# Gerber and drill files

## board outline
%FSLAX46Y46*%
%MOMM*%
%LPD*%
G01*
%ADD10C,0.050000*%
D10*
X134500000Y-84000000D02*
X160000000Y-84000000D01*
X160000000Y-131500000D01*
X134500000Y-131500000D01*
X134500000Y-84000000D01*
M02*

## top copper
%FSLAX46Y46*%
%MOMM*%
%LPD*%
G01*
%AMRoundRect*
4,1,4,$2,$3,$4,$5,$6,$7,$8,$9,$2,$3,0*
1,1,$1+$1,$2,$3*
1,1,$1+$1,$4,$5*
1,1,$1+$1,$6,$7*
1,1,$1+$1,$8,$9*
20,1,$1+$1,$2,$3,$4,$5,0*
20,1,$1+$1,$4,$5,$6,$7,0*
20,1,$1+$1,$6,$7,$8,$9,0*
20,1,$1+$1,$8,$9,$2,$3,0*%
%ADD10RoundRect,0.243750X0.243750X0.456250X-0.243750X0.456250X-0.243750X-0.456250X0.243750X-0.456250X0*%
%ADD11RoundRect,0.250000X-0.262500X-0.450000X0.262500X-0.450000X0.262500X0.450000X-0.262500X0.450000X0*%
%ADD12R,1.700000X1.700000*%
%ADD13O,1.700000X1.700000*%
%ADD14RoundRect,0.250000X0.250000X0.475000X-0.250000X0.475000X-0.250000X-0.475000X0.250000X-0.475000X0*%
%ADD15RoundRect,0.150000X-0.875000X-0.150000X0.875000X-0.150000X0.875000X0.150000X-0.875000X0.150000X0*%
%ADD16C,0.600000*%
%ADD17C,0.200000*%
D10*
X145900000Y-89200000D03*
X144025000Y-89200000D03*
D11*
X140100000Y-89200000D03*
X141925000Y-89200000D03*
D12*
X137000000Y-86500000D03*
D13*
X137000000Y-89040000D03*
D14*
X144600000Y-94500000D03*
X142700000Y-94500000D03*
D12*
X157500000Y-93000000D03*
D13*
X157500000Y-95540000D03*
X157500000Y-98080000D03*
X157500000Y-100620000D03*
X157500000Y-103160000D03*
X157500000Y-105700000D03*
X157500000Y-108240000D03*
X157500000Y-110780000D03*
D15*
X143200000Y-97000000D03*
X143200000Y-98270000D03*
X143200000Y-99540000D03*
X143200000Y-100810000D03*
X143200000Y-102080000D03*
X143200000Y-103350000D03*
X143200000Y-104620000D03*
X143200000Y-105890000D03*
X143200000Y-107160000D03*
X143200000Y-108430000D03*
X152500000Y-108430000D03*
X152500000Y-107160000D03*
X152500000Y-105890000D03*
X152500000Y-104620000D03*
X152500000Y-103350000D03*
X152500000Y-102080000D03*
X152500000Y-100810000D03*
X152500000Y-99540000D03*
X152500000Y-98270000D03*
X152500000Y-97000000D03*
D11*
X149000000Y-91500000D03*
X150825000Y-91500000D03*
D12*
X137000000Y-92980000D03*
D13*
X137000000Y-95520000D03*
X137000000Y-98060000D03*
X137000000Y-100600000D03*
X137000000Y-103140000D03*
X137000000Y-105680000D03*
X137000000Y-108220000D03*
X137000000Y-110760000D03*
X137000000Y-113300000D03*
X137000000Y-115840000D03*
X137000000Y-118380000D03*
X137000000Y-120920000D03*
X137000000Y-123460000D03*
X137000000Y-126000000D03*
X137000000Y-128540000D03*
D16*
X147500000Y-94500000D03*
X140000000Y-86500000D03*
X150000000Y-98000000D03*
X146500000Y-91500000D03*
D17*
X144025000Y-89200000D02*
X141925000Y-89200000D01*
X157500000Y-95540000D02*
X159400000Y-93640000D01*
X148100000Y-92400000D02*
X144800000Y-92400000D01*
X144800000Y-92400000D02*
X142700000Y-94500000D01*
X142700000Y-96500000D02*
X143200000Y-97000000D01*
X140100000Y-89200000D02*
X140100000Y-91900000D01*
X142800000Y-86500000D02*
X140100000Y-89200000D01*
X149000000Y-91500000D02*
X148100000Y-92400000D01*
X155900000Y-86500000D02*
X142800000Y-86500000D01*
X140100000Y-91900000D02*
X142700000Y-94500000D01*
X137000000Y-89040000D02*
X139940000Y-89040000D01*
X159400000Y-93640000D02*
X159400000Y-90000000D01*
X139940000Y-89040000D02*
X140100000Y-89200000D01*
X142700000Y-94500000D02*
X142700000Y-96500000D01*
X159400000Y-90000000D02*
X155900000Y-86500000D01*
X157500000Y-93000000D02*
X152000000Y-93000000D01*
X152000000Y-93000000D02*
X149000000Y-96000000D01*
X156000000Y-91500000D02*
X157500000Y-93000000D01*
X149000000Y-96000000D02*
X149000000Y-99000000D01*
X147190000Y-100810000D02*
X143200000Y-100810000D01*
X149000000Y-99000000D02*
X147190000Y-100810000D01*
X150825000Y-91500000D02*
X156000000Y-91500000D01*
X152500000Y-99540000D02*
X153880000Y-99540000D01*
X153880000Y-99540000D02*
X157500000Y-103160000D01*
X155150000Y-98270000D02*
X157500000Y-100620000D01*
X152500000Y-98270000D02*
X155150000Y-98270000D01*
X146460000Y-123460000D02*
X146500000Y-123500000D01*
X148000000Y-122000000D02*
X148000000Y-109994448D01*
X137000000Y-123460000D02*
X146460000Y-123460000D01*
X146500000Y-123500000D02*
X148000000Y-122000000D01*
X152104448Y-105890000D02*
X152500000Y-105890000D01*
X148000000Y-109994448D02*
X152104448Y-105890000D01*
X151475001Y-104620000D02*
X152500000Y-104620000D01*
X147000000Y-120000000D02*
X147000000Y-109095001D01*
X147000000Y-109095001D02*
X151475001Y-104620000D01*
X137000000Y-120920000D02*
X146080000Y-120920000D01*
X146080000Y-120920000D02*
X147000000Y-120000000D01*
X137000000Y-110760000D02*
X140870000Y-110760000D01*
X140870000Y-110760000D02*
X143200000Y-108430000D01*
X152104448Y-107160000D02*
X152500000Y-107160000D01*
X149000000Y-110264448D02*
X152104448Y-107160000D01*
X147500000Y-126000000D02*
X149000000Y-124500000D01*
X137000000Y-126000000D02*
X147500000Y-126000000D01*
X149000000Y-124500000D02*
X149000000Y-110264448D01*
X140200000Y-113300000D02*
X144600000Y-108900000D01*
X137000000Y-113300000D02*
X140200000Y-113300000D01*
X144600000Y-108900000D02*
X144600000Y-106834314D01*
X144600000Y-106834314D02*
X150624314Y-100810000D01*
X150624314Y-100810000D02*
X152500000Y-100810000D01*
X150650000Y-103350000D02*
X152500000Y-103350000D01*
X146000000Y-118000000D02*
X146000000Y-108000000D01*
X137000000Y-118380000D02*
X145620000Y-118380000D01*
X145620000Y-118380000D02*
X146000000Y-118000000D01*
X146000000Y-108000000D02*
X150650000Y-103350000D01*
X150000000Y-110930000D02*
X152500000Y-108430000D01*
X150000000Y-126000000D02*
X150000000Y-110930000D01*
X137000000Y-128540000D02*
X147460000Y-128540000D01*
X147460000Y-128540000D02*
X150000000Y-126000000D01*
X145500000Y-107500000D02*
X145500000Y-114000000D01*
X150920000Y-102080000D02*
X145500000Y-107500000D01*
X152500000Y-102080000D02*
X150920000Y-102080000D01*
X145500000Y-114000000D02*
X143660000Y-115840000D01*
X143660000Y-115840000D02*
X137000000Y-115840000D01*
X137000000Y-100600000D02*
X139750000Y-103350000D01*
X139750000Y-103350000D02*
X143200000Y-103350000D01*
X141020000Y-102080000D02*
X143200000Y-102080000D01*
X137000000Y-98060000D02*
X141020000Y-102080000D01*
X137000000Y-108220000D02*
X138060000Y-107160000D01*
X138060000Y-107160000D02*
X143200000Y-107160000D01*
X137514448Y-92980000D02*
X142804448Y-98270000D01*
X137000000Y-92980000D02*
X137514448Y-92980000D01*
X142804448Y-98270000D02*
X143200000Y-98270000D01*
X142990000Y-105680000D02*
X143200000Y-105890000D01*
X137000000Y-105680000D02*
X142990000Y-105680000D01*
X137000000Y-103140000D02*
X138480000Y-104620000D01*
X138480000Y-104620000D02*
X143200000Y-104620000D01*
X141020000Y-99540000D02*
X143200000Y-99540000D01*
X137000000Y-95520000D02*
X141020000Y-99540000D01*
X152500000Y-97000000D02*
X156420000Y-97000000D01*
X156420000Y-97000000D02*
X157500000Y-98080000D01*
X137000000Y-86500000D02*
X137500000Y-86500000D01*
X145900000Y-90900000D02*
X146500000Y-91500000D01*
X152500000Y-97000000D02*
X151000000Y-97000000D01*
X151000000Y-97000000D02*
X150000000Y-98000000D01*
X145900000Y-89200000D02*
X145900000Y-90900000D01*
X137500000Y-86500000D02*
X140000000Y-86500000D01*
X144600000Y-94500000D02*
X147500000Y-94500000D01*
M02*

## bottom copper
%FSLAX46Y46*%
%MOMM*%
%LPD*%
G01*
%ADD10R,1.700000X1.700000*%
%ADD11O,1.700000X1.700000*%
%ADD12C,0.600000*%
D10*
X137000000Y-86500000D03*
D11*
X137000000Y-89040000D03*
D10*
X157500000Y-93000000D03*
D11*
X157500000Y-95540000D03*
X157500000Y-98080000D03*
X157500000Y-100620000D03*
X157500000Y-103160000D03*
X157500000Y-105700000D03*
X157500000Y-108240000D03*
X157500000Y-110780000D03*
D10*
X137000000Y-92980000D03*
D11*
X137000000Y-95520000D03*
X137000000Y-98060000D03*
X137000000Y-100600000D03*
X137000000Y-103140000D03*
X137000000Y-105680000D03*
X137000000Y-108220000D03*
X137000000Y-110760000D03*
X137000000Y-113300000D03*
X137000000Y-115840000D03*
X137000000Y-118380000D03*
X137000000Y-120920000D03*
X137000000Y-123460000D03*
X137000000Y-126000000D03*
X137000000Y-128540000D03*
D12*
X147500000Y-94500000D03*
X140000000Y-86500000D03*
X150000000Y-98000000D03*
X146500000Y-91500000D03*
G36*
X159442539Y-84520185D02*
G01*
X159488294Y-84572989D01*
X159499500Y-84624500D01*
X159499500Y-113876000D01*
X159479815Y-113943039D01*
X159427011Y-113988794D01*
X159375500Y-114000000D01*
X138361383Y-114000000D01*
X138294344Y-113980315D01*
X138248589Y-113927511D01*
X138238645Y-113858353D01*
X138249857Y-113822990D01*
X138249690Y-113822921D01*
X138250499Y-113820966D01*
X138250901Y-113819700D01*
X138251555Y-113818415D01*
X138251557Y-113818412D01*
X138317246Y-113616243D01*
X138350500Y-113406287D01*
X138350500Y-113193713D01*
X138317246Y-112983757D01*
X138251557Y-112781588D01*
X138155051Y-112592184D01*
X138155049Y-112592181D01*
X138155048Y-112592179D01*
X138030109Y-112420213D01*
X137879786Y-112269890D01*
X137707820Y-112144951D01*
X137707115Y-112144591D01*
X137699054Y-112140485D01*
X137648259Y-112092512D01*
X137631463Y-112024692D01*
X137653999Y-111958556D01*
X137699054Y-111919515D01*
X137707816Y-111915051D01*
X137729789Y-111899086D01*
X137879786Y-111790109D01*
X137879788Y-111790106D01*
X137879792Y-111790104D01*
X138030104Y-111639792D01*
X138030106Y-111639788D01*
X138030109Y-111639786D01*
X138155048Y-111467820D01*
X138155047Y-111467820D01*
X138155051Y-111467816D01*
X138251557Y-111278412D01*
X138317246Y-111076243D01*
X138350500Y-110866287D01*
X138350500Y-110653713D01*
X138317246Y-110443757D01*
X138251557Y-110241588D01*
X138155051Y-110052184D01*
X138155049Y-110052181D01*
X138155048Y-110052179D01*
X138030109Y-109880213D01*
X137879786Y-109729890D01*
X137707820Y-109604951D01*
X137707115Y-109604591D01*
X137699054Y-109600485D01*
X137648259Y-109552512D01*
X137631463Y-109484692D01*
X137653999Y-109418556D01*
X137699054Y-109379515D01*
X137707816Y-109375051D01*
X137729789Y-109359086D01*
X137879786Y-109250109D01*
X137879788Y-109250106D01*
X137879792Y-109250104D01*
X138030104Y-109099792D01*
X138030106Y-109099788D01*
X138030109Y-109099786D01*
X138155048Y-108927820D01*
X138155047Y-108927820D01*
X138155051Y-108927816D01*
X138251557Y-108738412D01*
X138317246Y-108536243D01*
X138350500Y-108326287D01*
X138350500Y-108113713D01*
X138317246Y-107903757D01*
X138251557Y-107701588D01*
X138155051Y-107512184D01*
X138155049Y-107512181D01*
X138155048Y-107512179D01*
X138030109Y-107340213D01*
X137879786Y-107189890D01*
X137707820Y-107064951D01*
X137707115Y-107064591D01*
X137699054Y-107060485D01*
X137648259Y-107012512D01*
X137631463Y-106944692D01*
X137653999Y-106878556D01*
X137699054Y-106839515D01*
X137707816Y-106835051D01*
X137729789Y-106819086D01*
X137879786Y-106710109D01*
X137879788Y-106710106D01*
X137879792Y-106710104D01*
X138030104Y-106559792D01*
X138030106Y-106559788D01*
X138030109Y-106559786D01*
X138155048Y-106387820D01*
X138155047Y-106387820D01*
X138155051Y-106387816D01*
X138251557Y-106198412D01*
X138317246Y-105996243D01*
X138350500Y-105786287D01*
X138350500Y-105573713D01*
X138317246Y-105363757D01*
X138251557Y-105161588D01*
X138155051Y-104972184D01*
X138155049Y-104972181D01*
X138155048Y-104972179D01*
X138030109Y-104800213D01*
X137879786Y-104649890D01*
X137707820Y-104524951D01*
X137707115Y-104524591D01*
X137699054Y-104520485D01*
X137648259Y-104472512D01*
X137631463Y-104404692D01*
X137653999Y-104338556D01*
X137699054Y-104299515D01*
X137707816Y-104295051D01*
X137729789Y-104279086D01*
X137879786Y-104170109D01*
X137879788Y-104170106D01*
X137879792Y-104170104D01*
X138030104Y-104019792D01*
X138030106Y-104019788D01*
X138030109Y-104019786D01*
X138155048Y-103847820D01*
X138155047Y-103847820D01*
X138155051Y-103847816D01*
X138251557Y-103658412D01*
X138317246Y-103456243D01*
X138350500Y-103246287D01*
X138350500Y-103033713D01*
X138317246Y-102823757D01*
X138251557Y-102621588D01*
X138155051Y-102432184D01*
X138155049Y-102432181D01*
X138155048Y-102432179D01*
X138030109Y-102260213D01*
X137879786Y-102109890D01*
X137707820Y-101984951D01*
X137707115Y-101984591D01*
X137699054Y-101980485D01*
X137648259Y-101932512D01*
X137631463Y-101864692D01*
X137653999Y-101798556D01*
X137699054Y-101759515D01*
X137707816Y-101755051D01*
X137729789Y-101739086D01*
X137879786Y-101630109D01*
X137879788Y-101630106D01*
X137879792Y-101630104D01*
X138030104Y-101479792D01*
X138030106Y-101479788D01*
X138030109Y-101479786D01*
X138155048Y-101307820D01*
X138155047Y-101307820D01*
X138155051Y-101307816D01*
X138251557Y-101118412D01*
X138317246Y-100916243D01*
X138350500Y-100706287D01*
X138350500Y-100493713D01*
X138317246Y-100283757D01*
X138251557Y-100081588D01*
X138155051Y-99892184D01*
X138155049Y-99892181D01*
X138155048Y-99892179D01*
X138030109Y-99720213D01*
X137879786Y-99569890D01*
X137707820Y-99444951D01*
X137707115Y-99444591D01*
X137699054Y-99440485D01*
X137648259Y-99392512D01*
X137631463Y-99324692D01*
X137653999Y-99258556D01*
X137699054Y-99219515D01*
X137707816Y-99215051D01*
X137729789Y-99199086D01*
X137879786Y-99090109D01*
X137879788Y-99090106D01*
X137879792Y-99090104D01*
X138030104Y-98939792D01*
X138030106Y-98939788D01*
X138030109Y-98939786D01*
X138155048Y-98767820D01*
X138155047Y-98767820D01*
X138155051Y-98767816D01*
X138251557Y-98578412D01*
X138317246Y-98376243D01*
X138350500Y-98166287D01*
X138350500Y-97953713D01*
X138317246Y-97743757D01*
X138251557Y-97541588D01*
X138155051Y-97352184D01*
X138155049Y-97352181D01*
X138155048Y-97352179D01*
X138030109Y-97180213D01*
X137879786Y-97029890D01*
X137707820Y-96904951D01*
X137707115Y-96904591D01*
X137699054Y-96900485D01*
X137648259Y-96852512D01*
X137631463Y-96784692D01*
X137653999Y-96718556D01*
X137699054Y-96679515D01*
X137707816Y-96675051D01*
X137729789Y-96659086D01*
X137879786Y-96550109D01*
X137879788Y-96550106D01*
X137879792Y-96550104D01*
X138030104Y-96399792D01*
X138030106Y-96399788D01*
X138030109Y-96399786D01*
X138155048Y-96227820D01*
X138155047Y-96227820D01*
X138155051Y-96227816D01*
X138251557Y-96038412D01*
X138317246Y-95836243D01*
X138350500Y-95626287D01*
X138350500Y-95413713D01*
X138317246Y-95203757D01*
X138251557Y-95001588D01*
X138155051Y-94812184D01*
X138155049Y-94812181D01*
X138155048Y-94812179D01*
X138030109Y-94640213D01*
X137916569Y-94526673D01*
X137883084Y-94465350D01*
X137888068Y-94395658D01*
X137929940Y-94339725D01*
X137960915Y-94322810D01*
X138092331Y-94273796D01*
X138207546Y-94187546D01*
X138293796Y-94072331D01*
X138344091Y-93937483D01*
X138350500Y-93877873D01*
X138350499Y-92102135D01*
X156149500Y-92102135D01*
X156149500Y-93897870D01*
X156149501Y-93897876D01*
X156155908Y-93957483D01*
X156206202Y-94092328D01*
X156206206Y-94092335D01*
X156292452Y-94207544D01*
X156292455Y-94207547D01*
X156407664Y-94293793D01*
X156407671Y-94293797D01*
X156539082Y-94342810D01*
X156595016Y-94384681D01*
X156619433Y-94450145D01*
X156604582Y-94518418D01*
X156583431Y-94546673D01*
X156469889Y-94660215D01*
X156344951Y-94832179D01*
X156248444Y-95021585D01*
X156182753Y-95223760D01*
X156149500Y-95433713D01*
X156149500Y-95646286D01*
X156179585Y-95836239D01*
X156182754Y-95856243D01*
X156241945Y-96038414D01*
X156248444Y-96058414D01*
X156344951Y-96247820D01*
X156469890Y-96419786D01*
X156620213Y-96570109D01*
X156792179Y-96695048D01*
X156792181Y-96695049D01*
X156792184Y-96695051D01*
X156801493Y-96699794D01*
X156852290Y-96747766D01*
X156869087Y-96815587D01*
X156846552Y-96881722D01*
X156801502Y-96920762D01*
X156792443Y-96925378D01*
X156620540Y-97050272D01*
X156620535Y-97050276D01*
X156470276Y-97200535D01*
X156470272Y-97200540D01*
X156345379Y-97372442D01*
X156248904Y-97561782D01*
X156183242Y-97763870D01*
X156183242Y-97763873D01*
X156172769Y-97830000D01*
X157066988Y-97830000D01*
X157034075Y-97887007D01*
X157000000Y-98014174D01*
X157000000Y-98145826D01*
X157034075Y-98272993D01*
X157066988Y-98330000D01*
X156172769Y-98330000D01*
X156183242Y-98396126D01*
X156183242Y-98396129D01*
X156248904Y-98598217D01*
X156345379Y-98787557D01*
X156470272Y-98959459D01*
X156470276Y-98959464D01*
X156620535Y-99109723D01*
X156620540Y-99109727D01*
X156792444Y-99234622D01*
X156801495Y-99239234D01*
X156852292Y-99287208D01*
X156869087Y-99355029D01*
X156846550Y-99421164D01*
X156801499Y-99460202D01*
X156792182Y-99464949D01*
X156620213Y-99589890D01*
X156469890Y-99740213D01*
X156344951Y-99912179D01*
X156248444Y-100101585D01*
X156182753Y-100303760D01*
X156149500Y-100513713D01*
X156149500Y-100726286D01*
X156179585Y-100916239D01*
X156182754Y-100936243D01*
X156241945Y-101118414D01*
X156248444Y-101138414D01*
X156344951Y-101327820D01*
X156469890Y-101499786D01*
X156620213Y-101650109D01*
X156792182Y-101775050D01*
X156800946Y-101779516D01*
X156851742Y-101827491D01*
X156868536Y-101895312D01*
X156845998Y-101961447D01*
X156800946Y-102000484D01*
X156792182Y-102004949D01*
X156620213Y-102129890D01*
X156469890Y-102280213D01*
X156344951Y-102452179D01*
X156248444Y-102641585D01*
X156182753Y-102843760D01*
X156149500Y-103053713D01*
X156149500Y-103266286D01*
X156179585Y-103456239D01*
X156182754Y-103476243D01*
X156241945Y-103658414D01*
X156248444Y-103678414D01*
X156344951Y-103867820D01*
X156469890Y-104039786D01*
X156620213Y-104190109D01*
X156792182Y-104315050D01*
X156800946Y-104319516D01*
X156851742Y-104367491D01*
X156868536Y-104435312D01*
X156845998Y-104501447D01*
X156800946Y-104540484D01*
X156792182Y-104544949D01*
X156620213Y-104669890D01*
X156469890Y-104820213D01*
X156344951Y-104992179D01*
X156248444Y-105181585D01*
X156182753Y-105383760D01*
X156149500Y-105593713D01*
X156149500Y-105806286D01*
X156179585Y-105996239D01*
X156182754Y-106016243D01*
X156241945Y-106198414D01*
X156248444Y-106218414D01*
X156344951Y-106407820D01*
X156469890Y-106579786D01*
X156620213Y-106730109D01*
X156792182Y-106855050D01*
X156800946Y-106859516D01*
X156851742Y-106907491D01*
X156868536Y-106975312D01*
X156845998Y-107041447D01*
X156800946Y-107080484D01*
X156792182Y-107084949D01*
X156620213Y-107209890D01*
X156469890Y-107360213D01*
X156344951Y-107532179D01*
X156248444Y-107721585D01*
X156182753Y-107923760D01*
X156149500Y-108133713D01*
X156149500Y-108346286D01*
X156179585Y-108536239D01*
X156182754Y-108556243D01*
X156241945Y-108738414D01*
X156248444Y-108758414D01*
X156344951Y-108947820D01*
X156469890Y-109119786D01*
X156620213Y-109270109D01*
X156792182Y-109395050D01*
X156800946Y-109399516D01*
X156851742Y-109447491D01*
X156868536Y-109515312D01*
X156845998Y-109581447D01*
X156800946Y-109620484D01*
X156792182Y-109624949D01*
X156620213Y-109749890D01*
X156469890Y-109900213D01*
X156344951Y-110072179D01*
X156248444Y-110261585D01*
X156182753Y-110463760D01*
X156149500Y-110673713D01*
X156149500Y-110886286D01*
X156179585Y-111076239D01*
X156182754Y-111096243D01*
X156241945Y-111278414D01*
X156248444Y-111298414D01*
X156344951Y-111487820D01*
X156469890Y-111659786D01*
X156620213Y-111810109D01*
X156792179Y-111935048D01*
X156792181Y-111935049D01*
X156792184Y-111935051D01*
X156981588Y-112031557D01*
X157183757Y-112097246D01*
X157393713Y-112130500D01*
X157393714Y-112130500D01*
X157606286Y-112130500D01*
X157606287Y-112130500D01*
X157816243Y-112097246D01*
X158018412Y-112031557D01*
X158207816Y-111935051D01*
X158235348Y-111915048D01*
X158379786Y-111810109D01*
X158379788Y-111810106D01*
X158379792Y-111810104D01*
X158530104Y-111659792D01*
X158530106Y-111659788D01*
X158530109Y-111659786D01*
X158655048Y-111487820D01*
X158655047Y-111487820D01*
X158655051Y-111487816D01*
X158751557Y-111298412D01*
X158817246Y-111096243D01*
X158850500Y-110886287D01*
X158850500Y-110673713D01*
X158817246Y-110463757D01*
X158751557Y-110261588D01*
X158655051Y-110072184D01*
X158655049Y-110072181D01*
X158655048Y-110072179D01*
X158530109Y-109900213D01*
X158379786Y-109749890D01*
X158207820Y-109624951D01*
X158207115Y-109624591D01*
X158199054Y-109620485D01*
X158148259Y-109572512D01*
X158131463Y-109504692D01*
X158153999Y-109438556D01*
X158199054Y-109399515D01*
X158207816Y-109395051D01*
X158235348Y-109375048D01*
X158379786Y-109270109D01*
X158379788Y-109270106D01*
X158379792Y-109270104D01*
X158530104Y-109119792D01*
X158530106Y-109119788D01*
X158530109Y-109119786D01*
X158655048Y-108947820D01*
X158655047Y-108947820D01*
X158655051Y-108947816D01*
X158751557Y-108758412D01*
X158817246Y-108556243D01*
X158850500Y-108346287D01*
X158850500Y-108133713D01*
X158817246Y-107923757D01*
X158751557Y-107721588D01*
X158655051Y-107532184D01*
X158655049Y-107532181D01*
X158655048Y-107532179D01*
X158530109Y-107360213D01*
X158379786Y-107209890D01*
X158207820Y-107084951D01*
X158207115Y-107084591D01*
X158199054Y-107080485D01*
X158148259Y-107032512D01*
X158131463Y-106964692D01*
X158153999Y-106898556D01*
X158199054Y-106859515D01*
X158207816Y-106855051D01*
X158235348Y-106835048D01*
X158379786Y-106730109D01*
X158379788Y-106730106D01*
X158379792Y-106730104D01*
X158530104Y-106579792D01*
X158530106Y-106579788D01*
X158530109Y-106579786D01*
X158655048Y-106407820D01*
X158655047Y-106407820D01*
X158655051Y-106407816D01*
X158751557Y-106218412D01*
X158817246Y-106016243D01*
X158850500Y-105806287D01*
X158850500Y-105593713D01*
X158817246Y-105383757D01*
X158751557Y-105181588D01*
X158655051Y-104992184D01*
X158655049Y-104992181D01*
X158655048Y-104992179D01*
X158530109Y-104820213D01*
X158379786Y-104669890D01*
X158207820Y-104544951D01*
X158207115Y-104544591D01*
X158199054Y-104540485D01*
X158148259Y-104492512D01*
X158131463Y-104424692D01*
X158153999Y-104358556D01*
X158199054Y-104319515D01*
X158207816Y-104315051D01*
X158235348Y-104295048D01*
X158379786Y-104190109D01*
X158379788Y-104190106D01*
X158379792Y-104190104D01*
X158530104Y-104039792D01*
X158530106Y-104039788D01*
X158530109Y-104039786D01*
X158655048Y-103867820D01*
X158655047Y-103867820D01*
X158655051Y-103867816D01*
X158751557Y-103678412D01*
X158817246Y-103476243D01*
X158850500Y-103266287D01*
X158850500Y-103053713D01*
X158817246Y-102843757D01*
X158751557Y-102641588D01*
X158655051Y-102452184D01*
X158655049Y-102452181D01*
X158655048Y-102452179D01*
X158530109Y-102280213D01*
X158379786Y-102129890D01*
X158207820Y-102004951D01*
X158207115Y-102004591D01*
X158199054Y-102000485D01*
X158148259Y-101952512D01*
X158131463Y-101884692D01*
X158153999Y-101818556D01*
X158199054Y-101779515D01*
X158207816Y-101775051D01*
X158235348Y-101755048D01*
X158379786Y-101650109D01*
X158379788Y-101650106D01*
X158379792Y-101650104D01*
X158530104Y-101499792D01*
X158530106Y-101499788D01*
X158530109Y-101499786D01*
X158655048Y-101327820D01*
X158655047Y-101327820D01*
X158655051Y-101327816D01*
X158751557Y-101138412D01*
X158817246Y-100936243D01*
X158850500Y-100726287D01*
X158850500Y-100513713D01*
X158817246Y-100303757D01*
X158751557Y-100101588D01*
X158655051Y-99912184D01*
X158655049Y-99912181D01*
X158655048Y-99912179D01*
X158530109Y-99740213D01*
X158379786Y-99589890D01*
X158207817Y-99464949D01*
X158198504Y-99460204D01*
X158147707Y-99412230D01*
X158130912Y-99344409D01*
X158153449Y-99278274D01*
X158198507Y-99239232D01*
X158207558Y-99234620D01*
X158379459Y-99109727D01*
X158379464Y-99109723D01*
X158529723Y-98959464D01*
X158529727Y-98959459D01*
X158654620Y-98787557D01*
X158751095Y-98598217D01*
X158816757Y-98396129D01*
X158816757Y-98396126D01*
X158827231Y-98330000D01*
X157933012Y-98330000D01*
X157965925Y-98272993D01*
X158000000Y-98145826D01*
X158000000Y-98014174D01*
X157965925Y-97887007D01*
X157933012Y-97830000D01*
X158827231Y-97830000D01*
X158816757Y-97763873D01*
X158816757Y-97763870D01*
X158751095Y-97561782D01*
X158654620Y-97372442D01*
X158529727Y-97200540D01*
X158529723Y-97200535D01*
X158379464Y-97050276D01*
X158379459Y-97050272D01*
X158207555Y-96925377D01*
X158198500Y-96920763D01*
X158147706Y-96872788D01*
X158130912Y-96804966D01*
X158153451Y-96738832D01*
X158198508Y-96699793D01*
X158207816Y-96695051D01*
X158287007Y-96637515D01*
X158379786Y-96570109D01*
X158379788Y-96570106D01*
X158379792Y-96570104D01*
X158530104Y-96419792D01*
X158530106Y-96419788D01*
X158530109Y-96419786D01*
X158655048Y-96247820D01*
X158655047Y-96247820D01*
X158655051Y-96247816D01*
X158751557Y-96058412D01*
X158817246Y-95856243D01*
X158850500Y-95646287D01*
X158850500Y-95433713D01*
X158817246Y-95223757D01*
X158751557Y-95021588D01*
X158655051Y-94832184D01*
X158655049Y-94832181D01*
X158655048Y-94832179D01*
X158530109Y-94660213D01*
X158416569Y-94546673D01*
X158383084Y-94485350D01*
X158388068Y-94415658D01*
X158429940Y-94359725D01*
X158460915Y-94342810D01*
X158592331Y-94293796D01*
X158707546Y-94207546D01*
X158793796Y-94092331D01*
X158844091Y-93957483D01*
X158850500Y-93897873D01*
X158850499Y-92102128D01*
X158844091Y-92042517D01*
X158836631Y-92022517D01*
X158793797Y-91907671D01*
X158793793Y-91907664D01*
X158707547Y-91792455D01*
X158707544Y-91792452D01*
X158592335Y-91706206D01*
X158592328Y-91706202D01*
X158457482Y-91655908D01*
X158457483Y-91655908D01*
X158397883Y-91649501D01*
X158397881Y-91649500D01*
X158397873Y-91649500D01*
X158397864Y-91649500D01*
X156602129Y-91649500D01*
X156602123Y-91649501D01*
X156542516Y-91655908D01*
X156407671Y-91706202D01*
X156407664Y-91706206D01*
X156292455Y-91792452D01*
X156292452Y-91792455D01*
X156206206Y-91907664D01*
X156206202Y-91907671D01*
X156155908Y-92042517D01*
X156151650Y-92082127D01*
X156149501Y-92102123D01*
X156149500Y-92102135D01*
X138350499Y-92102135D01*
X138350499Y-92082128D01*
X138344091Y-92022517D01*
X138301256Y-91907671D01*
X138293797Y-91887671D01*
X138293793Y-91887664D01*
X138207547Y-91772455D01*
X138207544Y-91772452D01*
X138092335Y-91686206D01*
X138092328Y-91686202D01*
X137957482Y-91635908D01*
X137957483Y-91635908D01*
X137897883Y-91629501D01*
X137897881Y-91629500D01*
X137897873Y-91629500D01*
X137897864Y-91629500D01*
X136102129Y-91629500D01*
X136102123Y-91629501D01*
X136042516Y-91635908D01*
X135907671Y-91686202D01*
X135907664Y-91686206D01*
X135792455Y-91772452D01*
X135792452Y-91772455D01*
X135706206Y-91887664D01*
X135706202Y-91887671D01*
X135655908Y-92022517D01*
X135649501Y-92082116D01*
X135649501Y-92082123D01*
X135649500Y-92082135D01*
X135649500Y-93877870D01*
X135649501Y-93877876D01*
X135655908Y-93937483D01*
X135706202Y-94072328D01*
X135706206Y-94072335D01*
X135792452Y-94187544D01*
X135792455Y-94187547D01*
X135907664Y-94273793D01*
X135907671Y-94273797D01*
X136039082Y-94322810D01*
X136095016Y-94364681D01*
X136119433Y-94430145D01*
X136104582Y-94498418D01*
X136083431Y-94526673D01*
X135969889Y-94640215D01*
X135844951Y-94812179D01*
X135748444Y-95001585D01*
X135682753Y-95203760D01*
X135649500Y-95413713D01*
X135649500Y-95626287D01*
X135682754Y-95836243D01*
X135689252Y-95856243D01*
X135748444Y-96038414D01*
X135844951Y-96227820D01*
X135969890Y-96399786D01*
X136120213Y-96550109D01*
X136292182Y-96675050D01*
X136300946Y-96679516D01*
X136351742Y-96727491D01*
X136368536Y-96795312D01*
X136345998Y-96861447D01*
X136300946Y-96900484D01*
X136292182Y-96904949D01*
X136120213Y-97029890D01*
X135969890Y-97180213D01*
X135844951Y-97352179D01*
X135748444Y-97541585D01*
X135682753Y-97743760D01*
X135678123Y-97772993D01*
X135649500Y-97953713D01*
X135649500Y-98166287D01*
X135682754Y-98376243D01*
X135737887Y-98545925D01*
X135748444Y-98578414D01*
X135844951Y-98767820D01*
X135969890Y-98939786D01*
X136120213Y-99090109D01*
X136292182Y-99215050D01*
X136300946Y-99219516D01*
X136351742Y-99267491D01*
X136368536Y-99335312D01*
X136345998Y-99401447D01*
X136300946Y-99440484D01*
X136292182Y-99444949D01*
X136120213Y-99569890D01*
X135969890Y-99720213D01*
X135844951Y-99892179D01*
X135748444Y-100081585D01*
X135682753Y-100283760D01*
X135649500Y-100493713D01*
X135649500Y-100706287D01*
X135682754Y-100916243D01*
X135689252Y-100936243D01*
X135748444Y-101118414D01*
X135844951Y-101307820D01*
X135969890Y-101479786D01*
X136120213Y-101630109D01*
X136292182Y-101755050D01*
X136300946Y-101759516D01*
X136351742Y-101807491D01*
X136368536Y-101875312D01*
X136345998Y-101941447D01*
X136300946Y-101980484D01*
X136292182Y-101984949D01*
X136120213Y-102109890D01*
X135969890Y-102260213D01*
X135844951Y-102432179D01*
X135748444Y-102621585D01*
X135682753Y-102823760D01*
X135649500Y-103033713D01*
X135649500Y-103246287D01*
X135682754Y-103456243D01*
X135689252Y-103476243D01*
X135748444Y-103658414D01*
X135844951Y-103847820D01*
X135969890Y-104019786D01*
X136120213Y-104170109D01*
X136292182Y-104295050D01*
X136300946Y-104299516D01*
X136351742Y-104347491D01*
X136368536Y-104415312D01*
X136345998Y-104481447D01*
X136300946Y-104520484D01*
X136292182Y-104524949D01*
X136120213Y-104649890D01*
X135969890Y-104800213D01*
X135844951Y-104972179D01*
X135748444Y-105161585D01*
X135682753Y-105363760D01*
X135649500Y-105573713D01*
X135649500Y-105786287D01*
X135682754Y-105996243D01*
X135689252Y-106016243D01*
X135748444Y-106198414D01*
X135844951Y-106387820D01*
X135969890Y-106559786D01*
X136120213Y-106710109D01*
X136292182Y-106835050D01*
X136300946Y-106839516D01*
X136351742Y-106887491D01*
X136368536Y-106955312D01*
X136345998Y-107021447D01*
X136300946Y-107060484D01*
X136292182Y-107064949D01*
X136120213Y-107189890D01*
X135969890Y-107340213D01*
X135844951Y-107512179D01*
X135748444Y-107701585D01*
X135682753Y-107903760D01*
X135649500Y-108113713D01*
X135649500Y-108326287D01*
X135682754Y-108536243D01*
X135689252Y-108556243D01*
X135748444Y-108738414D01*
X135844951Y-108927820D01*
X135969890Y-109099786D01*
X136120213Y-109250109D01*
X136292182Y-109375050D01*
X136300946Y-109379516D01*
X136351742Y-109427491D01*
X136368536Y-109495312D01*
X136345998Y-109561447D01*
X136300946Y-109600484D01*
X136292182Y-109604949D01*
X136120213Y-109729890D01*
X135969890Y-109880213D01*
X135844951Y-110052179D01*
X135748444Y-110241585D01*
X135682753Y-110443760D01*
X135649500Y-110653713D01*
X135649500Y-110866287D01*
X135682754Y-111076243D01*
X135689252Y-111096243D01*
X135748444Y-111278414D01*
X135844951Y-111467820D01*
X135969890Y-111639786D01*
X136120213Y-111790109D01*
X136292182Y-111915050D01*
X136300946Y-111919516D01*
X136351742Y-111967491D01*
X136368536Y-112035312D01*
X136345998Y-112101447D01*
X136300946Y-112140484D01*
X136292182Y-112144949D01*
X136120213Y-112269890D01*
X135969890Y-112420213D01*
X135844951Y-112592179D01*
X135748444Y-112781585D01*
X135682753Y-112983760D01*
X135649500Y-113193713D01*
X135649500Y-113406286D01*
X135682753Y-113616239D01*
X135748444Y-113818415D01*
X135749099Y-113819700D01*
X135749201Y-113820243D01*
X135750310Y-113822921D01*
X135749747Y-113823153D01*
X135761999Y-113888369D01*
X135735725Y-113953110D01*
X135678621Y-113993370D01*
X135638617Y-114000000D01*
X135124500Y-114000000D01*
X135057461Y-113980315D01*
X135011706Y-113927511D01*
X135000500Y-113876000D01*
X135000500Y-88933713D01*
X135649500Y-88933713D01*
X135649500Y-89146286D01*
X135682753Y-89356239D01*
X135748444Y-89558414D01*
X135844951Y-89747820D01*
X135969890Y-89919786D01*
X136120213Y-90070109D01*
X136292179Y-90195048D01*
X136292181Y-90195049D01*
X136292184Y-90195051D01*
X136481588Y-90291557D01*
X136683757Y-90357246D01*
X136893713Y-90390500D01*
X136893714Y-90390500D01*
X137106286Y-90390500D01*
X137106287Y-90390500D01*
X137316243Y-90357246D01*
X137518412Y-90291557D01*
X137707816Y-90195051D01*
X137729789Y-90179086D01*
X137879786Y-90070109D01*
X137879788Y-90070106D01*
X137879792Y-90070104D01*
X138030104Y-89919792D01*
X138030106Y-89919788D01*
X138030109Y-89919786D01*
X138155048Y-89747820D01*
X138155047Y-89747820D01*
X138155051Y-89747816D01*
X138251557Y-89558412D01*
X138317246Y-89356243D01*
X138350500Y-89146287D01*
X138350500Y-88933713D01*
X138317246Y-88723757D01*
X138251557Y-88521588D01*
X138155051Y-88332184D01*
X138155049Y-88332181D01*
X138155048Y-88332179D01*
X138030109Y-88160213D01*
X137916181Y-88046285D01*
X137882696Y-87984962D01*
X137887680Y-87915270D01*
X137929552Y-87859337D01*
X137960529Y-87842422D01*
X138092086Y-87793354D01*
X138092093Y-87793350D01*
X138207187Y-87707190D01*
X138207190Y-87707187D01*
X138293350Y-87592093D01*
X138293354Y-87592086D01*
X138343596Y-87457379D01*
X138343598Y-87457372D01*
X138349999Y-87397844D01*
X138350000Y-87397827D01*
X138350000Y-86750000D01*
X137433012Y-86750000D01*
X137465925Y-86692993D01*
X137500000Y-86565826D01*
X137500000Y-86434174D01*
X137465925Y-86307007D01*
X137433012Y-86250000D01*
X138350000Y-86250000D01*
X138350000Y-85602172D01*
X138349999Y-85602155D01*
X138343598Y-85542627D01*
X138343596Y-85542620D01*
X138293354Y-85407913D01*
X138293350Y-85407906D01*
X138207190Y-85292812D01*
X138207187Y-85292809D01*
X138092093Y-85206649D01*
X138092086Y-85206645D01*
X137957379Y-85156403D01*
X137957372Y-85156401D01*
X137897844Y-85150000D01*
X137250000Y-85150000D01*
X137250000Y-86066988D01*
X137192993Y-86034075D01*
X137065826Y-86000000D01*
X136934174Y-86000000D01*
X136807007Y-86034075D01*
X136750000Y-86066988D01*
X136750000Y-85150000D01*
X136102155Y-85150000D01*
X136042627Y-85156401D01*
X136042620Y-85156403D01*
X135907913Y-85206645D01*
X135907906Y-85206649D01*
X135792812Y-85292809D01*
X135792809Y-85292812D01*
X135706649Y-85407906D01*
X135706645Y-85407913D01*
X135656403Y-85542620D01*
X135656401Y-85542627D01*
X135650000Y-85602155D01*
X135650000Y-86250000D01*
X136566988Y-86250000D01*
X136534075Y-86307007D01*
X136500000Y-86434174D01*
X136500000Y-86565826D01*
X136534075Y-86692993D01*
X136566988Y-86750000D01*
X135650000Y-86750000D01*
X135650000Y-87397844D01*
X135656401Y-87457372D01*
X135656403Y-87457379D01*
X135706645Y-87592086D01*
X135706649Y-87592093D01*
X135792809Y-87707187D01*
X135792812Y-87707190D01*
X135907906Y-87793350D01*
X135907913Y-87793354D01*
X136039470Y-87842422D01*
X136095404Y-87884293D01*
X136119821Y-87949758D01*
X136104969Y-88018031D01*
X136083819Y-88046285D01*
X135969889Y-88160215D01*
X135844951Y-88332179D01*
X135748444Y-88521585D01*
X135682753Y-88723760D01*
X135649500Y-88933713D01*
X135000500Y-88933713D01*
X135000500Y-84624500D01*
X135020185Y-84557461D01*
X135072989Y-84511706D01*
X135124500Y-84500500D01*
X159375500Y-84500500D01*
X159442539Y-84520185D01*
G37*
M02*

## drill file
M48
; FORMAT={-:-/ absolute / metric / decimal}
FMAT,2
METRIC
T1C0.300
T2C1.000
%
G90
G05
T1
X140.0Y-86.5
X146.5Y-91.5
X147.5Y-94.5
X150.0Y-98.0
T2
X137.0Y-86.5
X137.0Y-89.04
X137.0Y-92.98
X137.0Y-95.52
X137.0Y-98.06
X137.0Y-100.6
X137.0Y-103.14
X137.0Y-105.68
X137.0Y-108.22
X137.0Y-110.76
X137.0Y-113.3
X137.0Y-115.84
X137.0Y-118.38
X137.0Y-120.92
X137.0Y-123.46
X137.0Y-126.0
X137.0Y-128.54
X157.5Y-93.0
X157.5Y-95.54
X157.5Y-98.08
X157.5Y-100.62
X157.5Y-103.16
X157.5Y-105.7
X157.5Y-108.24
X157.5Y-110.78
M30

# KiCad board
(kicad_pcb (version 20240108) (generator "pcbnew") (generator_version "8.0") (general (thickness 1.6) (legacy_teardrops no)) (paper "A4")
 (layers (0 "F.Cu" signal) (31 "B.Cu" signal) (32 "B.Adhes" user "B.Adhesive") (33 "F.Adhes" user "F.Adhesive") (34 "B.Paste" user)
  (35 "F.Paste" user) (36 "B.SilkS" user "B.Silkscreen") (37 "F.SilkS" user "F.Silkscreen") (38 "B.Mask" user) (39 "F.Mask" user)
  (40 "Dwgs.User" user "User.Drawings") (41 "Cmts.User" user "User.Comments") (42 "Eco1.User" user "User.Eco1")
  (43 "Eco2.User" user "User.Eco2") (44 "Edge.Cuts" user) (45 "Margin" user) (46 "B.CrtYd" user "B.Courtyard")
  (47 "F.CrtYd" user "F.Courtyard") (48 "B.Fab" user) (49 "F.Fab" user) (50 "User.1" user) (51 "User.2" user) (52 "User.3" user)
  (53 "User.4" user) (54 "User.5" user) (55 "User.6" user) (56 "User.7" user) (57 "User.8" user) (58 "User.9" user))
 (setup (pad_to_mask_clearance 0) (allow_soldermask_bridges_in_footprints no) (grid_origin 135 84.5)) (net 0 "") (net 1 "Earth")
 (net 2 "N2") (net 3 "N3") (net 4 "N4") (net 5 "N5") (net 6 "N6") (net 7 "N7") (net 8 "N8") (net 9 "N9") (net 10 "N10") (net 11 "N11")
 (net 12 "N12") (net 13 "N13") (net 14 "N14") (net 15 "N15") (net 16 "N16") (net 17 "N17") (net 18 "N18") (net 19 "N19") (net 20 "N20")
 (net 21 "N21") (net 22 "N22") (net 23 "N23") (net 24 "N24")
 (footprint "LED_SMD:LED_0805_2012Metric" (layer "F.Cu") (at 144.9625 89.2 180)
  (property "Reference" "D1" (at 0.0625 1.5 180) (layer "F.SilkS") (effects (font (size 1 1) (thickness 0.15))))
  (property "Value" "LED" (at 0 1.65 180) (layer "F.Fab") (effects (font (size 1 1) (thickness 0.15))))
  (pad "1" smd roundrect (at -0.9375 0 180) (size 0.975 1.4) (layers "F.Cu" "F.Paste" "F.Mask") (roundrect_rratio 0.25) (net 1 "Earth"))
  (pad "2" smd roundrect (at 0.9375 0 180) (size 0.975 1.4) (layers "F.Cu" "F.Paste" "F.Mask") (roundrect_rratio 0.25) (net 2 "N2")))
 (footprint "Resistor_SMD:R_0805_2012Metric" (layer "F.Cu") (at 141.0125 89.2)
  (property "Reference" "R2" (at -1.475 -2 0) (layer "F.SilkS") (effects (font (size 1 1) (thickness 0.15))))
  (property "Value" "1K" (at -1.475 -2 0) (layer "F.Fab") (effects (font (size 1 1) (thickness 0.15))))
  (pad "1" smd roundrect (at -0.9125 0) (size 1.025 1.4) (layers "F.Cu" "F.Paste" "F.Mask") (roundrect_rratio 0.243902439) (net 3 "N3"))
  (pad "2" smd roundrect (at 0.9125 0) (size 1.025 1.4) (layers "F.Cu" "F.Paste" "F.Mask") (roundrect_rratio 0.243902439) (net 2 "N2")))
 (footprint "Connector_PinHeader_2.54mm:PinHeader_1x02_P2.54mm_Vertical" (layer "F.Cu") (at 137 86.5)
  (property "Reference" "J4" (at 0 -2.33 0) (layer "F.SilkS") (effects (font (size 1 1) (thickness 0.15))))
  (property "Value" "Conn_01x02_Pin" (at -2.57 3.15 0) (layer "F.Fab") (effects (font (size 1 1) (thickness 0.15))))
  (pad "1" thru_hole rect (at 0 0) (size 1.7 1.7) (drill 1) (layers "*.Cu" "*.Mask") (remove_unused_layers no) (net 1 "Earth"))
  (pad "2" thru_hole oval (at 0 2.54) (size 1.7 1.7) (drill 1) (layers "*.Cu" "*.Mask") (remove_unused_layers no) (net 3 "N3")))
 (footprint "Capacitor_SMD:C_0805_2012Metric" (layer "F.Cu") (at 143.65 94.5 180)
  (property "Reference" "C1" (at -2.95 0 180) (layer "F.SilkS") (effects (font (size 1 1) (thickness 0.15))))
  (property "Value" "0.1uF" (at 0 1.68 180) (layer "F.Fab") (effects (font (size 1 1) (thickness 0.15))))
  (pad "1" smd roundrect (at -0.95 0 180) (size 1 1.45) (layers "F.Cu" "F.Paste" "F.Mask") (roundrect_rratio 0.25) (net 1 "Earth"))
  (pad "2" smd roundrect (at 0.95 0 180) (size 1 1.45) (layers "F.Cu" "F.Paste" "F.Mask") (roundrect_rratio 0.25) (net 3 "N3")))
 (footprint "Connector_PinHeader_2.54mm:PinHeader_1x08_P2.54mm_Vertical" (layer "F.Cu") (at 157.5 93)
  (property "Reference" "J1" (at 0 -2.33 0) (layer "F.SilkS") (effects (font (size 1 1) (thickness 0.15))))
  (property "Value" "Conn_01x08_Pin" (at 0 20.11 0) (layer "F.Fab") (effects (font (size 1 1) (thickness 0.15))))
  (pad "1" thru_hole rect (at 0 0) (size 1.7 1.7) (drill 1) (layers "*.Cu" "*.Mask") (remove_unused_layers no) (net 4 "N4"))
  (pad "2" thru_hole oval (at 0 2.54) (size 1.7 1.7) (drill 1) (layers "*.Cu" "*.Mask") (remove_unused_layers no) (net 3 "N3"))
  (pad "3" thru_hole oval (at 0 5.08) (size 1.7 1.7) (drill 1) (layers "*.Cu" "*.Mask") (remove_unused_layers no) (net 1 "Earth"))
  (pad "4" thru_hole oval (at 0 7.62) (size 1.7 1.7) (drill 1) (layers "*.Cu" "*.Mask") (remove_unused_layers no) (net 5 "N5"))
  (pad "5" thru_hole oval (at 0 10.16) (size 1.7 1.7) (drill 1) (layers "*.Cu" "*.Mask") (remove_unused_layers no) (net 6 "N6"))
  (pad "6" thru_hole oval (at 0 12.7) (size 1.7 1.7) (drill 1) (layers "*.Cu" "*.Mask") (remove_unused_layers no) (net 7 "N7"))
  (pad "7" thru_hole oval (at 0 15.24) (size 1.7 1.7) (drill 1) (layers "*.Cu" "*.Mask") (remove_unused_layers no) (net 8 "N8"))
  (pad "8" thru_hole oval (at 0 17.78) (size 1.7 1.7) (drill 1) (layers "*.Cu" "*.Mask") (remove_unused_layers no) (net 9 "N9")))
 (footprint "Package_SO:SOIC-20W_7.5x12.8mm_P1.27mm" (layer "F.Cu") (at 147.85 102.715)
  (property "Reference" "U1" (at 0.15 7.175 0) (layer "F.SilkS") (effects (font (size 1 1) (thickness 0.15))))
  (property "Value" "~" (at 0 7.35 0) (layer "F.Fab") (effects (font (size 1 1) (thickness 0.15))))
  (pad "1" smd roundrect (at -4.65 -5.715) (size 2.05 0.6) (layers "F.Cu" "F.Paste" "F.Mask") (roundrect_rratio 0.25) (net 3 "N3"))
  (pad "2" smd roundrect (at -4.65 -4.445) (size 2.05 0.6) (layers "F.Cu" "F.Paste" "F.Mask") (roundrect_rratio 0.25) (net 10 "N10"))
  (pad "3" smd roundrect (at -4.65 -3.175) (size 2.05 0.6) (layers "F.Cu" "F.Paste" "F.Mask") (roundrect_rratio 0.25) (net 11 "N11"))
  (pad "4" smd roundrect (at -4.65 -1.905) (size 2.05 0.6) (layers "F.Cu" "F.Paste" "F.Mask") (roundrect_rratio 0.25) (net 4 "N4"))
  (pad "5" smd roundrect (at -4.65 -0.635) (size 2.05 0.6) (layers "F.Cu" "F.Paste" "F.Mask") (roundrect_rratio 0.25) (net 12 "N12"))
  (pad "6" smd roundrect (at -4.65 0.635) (size 2.05 0.6) (layers "F.Cu" "F.Paste" "F.Mask") (roundrect_rratio 0.25) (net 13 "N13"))
  (pad "7" smd roundrect (at -4.65 1.905) (size 2.05 0.6) (layers "F.Cu" "F.Paste" "F.Mask") (roundrect_rratio 0.25) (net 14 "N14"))
  (pad "8" smd roundrect (at -4.65 3.175) (size 2.05 0.6) (layers "F.Cu" "F.Paste" "F.Mask") (roundrect_rratio 0.25) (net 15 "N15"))
  (pad "9" smd roundrect (at -4.65 4.445) (size 2.05 0.6) (layers "F.Cu" "F.Paste" "F.Mask") (roundrect_rratio 0.25) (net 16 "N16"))
  (pad "10" smd roundrect (at -4.65 5.715) (size 2.05 0.6) (layers "F.Cu" "F.Paste" "F.Mask") (roundrect_rratio 0.25) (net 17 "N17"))
  (pad "11" smd roundrect (at 4.65 5.715) (size 2.05 0.6) (layers "F.Cu" "F.Paste" "F.Mask") (roundrect_rratio 0.25) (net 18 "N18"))
  (pad "12" smd roundrect (at 4.65 4.445) (size 2.05 0.6) (layers "F.Cu" "F.Paste" "F.Mask") (roundrect_rratio 0.25) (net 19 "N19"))
  (pad "13" smd roundrect (at 4.65 3.175) (size 2.05 0.6) (layers "F.Cu" "F.Paste" "F.Mask") (roundrect_rratio 0.25) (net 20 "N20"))
  (pad "14" smd roundrect (at 4.65 1.905) (size 2.05 0.6) (layers "F.Cu" "F.Paste" "F.Mask") (roundrect_rratio 0.25) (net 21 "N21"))
  (pad "15" smd roundrect (at 4.65 0.635) (size 2.05 0.6) (layers "F.Cu" "F.Paste" "F.Mask") (roundrect_rratio 0.25) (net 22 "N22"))
  (pad "16" smd roundrect (at 4.65 -0.635) (size 2.05 0.6) (layers "F.Cu" "F.Paste" "F.Mask") (roundrect_rratio 0.25) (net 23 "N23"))
  (pad "17" smd roundrect (at 4.65 -1.905) (size 2.05 0.6) (layers "F.Cu" "F.Paste" "F.Mask") (roundrect_rratio 0.25) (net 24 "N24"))
  (pad "18" smd roundrect (at 4.65 -3.175) (size 2.05 0.6) (layers "F.Cu" "F.Paste" "F.Mask") (roundrect_rratio 0.25) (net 6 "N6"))
  (pad "19" smd roundrect (at 4.65 -4.445) (size 2.05 0.6) (layers "F.Cu" "F.Paste" "F.Mask") (roundrect_rratio 0.25) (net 5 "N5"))
  (pad "20" smd roundrect (at 4.65 -5.715) (size 2.05 0.6) (layers "F.Cu" "F.Paste" "F.Mask") (roundrect_rratio 0.25) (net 1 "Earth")))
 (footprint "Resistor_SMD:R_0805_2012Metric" (layer "F.Cu") (at 149.9125 91.5)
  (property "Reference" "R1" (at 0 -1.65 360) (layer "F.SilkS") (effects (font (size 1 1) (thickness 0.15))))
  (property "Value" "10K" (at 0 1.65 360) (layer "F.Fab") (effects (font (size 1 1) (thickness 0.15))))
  (pad "1" smd roundrect (at -0.9125 0) (size 1.025 1.4) (layers "F.Cu" "F.Paste" "F.Mask") (roundrect_rratio 0.243902439) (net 3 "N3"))
  (pad "2" smd roundrect (at 0.9125 0) (size 1.025 1.4) (layers "F.Cu" "F.Paste" "F.Mask") (roundrect_rratio 0.243902439) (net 4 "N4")))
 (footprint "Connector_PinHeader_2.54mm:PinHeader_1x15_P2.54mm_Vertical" (layer "B.Cu") (at 137 92.98 180)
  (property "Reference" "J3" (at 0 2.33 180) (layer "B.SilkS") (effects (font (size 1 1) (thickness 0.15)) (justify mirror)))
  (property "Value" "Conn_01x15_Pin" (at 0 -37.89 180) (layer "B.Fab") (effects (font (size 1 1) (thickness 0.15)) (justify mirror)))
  (pad "1" thru_hole rect (at 0 0 180) (size 1.7 1.7) (drill 1) (layers "*.Cu" "*.Mask") (remove_unused_layers no) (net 10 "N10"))
  (pad "2" thru_hole oval (at 0 -2.54 180) (size 1.7 1.7) (drill 1) (layers "*.Cu" "*.Mask") (remove_unused_layers no) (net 11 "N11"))
  (pad "3" thru_hole oval (at 0 -5.08 180) (size 1.7 1.7) (drill 1) (layers "*.Cu" "*.Mask") (remove_unused_layers no) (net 12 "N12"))
  (pad "4" thru_hole oval (at 0 -7.62 180) (size 1.7 1.7) (drill 1) (layers "*.Cu" "*.Mask") (remove_unused_layers no) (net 13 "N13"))
  (pad "5" thru_hole oval (at 0 -10.16 180) (size 1.7 1.7) (drill 1) (layers "*.Cu" "*.Mask") (remove_unused_layers no) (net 14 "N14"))
  (pad "6" thru_hole oval (at 0 -12.7 180) (size 1.7 1.7) (drill 1) (layers "*.Cu" "*.Mask") (remove_unused_layers no) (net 15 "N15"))
  (pad "7" thru_hole oval (at 0 -15.24 180) (size 1.7 1.7) (drill 1) (layers "*.Cu" "*.Mask") (remove_unused_layers no) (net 16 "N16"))
  (pad "8" thru_hole oval (at 0 -17.78 180) (size 1.7 1.7) (drill 1) (layers "*.Cu" "*.Mask") (remove_unused_layers no) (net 17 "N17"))
  (pad "9" thru_hole oval (at 0 -20.32 180) (size 1.7 1.7) (drill 1) (layers "*.Cu" "*.Mask") (remove_unused_layers no) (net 24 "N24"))
  (pad "10" thru_hole oval (at 0 -22.86 180) (size 1.7 1.7) (drill 1) (layers "*.Cu" "*.Mask") (remove_unused_layers no) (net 23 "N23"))
  (pad "11" thru_hole oval (at 0 -25.4 180) (size 1.7 1.7) (drill 1) (layers "*.Cu" "*.Mask") (remove_unused_layers no) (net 22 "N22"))
  (pad "12" thru_hole oval (at 0 -27.94 180) (size 1.7 1.7) (drill 1) (layers "*.Cu" "*.Mask") (remove_unused_layers no) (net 21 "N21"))
  (pad "13" thru_hole oval (at 0 -30.48 180) (size 1.7 1.7) (drill 1) (layers "*.Cu" "*.Mask") (remove_unused_layers no) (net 20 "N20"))
  (pad "14" thru_hole oval (at 0 -33.02 180) (size 1.7 1.7) (drill 1) (layers "*.Cu" "*.Mask") (remove_unused_layers no) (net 19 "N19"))
  (pad "15" thru_hole oval (at 0 -35.56 180) (size 1.7 1.7) (drill 1) (layers "*.Cu" "*.Mask") (remove_unused_layers no) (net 18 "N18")))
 (gr_rect (start 134.5 84) (end 160 131.5) (stroke (width 0.05) (type default)) (fill none) (layer "Edge.Cuts"))
 (segment (start 144.025 89.2) (end 141.925 89.2) (width 0.2) (layer "F.Cu") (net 2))
 (segment (start 157.5 95.54) (end 159.4 93.64) (width 0.2) (layer "F.Cu") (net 3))
 (segment (start 148.1 92.4) (end 144.8 92.4) (width 0.2) (layer "F.Cu") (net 3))
 (segment (start 144.8 92.4) (end 142.7 94.5) (width 0.2) (layer "F.Cu") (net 3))
 (segment (start 142.7 96.5) (end 143.2 97) (width 0.2) (layer "F.Cu") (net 3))
 (segment (start 140.1 89.2) (end 140.1 91.9) (width 0.2) (layer "F.Cu") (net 3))
 (segment (start 142.8 86.5) (end 140.1 89.2) (width 0.2) (layer "F.Cu") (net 3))
 (segment (start 149 91.5) (end 148.1 92.4) (width 0.2) (layer "F.Cu") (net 3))
 (segment (start 155.9 86.5) (end 142.8 86.5) (width 0.2) (layer "F.Cu") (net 3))
 (segment (start 140.1 91.9) (end 142.7 94.5) (width 0.2) (layer "F.Cu") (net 3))
 (segment (start 137 89.04) (end 139.94 89.04) (width 0.2) (layer "F.Cu") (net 3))
 (segment (start 159.4 93.64) (end 159.4 90) (width 0.2) (layer "F.Cu") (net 3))
 (segment (start 139.94 89.04) (end 140.1 89.2) (width 0.2) (layer "F.Cu") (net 3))
 (segment (start 142.7 94.5) (end 142.7 96.5) (width 0.2) (layer "F.Cu") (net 3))
 (segment (start 159.4 90) (end 155.9 86.5) (width 0.2) (layer "F.Cu") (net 3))
 (segment (start 157.5 93) (end 152 93) (width 0.2) (layer "F.Cu") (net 4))
 (segment (start 152 93) (end 149 96) (width 0.2) (layer "F.Cu") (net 4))
 (segment (start 156 91.5) (end 157.5 93) (width 0.2) (layer "F.Cu") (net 4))
 (segment (start 149 96) (end 149 99) (width 0.2) (layer "F.Cu") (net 4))
 (segment (start 147.19 100.81) (end 143.2 100.81) (width 0.2) (layer "F.Cu") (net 4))
 (segment (start 149 99) (end 147.19 100.81) (width 0.2) (layer "F.Cu") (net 4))
 (segment (start 150.825 91.5) (end 156 91.5) (width 0.2) (layer "F.Cu") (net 4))
 (segment (start 152.5 99.54) (end 153.88 99.54) (width 0.2) (layer "F.Cu") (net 6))
 (segment (start 153.88 99.54) (end 157.5 103.16) (width 0.2) (layer "F.Cu") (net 6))
 (segment (start 155.15 98.27) (end 157.5 100.62) (width 0.2) (layer "F.Cu") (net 5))
 (segment (start 152.5 98.27) (end 155.15 98.27) (width 0.2) (layer "F.Cu") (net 5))
 (segment (start 146.46 123.46) (end 146.5 123.5) (width 0.2) (layer "F.Cu") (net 20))
 (segment (start 148 122) (end 148 109.994448) (width 0.2) (layer "F.Cu") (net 20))
 (segment (start 137 123.46) (end 146.46 123.46) (width 0.2) (layer "F.Cu") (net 20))
 (segment (start 146.5 123.5) (end 148 122) (width 0.2) (layer "F.Cu") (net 20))
 (segment (start 152.104448 105.89) (end 152.5 105.89) (width 0.2) (layer "F.Cu") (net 20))
 (segment (start 148 109.994448) (end 152.104448 105.89) (width 0.2) (layer "F.Cu") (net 20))
 (segment (start 151.475001 104.62) (end 152.5 104.62) (width 0.2) (layer "F.Cu") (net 21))
 (segment (start 147 120) (end 147 109.095001) (width 0.2) (layer "F.Cu") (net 21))
 (segment (start 147 109.095001) (end 151.475001 104.62) (width 0.2) (layer "F.Cu") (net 21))
 (segment (start 137 120.92) (end 146.08 120.92) (width 0.2) (layer "F.Cu") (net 21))
 (segment (start 146.08 120.92) (end 147 120) (width 0.2) (layer "F.Cu") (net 21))
 (segment (start 137 110.76) (end 140.87 110.76) (width 0.2) (layer "F.Cu") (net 17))
 (segment (start 140.87 110.76) (end 143.2 108.43) (width 0.2) (layer "F.Cu") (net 17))
 (segment (start 152.104448 107.16) (end 152.5 107.16) (width 0.2) (layer "F.Cu") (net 19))
 (segment (start 149 110.264448) (end 152.104448 107.16) (width 0.2) (layer "F.Cu") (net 19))
 (segment (start 147.5 126) (end 149 124.5) (width 0.2) (layer "F.Cu") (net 19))
 (segment (start 137 126) (end 147.5 126) (width 0.2) (layer "F.Cu") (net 19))
 (segment (start 149 124.5) (end 149 110.264448) (width 0.2) (layer "F.Cu") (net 19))
 (segment (start 140.2 113.3) (end 144.6 108.9) (width 0.2) (layer "F.Cu") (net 24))
 (segment (start 137 113.3) (end 140.2 113.3) (width 0.2) (layer "F.Cu") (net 24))
 (segment (start 144.6 108.9) (end 144.6 106.834314) (width 0.2) (layer "F.Cu") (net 24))
 (segment (start 144.6 106.834314) (end 150.624314 100.81) (width 0.2) (layer "F.Cu") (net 24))
 (segment (start 150.624314 100.81) (end 152.5 100.81) (width 0.2) (layer "F.Cu") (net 24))
 (segment (start 150.65 103.35) (end 152.5 103.35) (width 0.2) (layer "F.Cu") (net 22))
 (segment (start 146 118) (end 146 108) (width 0.2) (layer "F.Cu") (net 22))
 (segment (start 137 118.38) (end 145.62 118.38) (width 0.2) (layer "F.Cu") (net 22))
 (segment (start 145.62 118.38) (end 146 118) (width 0.2) (layer "F.Cu") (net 22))
 (segment (start 146 108) (end 150.65 103.35) (width 0.2) (layer "F.Cu") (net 22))
 (segment (start 150 110.93) (end 152.5 108.43) (width 0.2) (layer "F.Cu") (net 18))
 (segment (start 150 126) (end 150 110.93) (width 0.2) (layer "F.Cu") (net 18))
 (segment (start 137 128.54) (end 147.46 128.54) (width 0.2) (layer "F.Cu") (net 18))
 (segment (start 147.46 128.54) (end 150 126) (width 0.2) (layer "F.Cu") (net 18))
 (segment (start 145.5 107.5) (end 145.5 114) (width 0.2) (layer "F.Cu") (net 23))
 (segment (start 150.92 102.08) (end 145.5 107.5) (width 0.2) (layer "F.Cu") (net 23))
 (segment (start 152.5 102.08) (end 150.92 102.08) (width 0.2) (layer "F.Cu") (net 23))
 (segment (start 145.5 114) (end 143.66 115.84) (width 0.2) (layer "F.Cu") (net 23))
 (segment (start 143.66 115.84) (end 137 115.84) (width 0.2) (layer "F.Cu") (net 23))
 (segment (start 137 100.6) (end 139.75 103.35) (width 0.2) (layer "F.Cu") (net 13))
 (segment (start 139.75 103.35) (end 143.2 103.35) (width 0.2) (layer "F.Cu") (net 13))
 (segment (start 141.02 102.08) (end 143.2 102.08) (width 0.2) (layer "F.Cu") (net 12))
 (segment (start 137 98.06) (end 141.02 102.08) (width 0.2) (layer "F.Cu") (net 12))
 (segment (start 137 108.22) (end 138.06 107.16) (width 0.2) (layer "F.Cu") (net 16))
 (segment (start 138.06 107.16) (end 143.2 107.16) (width 0.2) (layer "F.Cu") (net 16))
 (segment (start 137.514448 92.98) (end 142.804448 98.27) (width 0.2) (layer "F.Cu") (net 10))
 (segment (start 137 92.98) (end 137.514448 92.98) (width 0.2) (layer "F.Cu") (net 10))
 (segment (start 142.804448 98.27) (end 143.2 98.27) (width 0.2) (layer "F.Cu") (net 10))
 (segment (start 142.99 105.68) (end 143.2 105.89) (width 0.2) (layer "F.Cu") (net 15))
 (segment (start 137 105.68) (end 142.99 105.68) (width 0.2) (layer "F.Cu") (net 15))
 (segment (start 137 103.14) (end 138.48 104.62) (width 0.2) (layer "F.Cu") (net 14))
 (segment (start 138.48 104.62) (end 143.2 104.62) (width 0.2) (layer "F.Cu") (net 14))
 (segment (start 141.02 99.54) (end 143.2 99.54) (width 0.2) (layer "F.Cu") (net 11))
 (segment (start 137 95.52) (end 141.02 99.54) (width 0.2) (layer "F.Cu") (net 11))
 (segment (start 152.5 97) (end 156.42 97) (width 0.2) (layer "F.Cu") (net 1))
 (segment (start 156.42 97) (end 157.5 98.08) (width 0.2) (layer "F.Cu") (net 1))
 (segment (start 137 86.5) (end 137.5 86.5) (width 0.2) (layer "F.Cu") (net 1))
 (segment (start 145.9 90.9) (end 146.5 91.5) (width 0.2) (layer "F.Cu") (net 1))
 (segment (start 152.5 97) (end 151 97) (width 0.2) (layer "F.Cu") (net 1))
 (segment (start 151 97) (end 150 98) (width 0.2) (layer "F.Cu") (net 1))
 (segment (start 145.9 89.2) (end 145.9 90.9) (width 0.2) (layer "F.Cu") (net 1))
 (segment (start 137.5 86.5) (end 140 86.5) (width 0.2) (layer "F.Cu") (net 1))
 (segment (start 144.6 94.5) (end 147.5 94.5) (width 0.2) (layer "F.Cu") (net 1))
 (via (at 147.5 94.5) (size 0.6) (drill 0.3) (layers "F.Cu" "B.Cu") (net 1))
 (via (at 140 86.5) (size 0.6) (drill 0.3) (layers "F.Cu" "B.Cu") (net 1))
 (via (at 150 98) (size 0.6) (drill 0.3) (layers "F.Cu" "B.Cu") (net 1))
 (via (at 146.5 91.5) (size 0.6) (drill 0.3) (layers "F.Cu" "B.Cu") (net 1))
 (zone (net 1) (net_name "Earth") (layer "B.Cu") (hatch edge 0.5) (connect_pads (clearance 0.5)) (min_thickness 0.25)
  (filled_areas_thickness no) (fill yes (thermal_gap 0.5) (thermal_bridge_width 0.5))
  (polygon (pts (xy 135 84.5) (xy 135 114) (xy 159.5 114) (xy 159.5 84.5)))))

